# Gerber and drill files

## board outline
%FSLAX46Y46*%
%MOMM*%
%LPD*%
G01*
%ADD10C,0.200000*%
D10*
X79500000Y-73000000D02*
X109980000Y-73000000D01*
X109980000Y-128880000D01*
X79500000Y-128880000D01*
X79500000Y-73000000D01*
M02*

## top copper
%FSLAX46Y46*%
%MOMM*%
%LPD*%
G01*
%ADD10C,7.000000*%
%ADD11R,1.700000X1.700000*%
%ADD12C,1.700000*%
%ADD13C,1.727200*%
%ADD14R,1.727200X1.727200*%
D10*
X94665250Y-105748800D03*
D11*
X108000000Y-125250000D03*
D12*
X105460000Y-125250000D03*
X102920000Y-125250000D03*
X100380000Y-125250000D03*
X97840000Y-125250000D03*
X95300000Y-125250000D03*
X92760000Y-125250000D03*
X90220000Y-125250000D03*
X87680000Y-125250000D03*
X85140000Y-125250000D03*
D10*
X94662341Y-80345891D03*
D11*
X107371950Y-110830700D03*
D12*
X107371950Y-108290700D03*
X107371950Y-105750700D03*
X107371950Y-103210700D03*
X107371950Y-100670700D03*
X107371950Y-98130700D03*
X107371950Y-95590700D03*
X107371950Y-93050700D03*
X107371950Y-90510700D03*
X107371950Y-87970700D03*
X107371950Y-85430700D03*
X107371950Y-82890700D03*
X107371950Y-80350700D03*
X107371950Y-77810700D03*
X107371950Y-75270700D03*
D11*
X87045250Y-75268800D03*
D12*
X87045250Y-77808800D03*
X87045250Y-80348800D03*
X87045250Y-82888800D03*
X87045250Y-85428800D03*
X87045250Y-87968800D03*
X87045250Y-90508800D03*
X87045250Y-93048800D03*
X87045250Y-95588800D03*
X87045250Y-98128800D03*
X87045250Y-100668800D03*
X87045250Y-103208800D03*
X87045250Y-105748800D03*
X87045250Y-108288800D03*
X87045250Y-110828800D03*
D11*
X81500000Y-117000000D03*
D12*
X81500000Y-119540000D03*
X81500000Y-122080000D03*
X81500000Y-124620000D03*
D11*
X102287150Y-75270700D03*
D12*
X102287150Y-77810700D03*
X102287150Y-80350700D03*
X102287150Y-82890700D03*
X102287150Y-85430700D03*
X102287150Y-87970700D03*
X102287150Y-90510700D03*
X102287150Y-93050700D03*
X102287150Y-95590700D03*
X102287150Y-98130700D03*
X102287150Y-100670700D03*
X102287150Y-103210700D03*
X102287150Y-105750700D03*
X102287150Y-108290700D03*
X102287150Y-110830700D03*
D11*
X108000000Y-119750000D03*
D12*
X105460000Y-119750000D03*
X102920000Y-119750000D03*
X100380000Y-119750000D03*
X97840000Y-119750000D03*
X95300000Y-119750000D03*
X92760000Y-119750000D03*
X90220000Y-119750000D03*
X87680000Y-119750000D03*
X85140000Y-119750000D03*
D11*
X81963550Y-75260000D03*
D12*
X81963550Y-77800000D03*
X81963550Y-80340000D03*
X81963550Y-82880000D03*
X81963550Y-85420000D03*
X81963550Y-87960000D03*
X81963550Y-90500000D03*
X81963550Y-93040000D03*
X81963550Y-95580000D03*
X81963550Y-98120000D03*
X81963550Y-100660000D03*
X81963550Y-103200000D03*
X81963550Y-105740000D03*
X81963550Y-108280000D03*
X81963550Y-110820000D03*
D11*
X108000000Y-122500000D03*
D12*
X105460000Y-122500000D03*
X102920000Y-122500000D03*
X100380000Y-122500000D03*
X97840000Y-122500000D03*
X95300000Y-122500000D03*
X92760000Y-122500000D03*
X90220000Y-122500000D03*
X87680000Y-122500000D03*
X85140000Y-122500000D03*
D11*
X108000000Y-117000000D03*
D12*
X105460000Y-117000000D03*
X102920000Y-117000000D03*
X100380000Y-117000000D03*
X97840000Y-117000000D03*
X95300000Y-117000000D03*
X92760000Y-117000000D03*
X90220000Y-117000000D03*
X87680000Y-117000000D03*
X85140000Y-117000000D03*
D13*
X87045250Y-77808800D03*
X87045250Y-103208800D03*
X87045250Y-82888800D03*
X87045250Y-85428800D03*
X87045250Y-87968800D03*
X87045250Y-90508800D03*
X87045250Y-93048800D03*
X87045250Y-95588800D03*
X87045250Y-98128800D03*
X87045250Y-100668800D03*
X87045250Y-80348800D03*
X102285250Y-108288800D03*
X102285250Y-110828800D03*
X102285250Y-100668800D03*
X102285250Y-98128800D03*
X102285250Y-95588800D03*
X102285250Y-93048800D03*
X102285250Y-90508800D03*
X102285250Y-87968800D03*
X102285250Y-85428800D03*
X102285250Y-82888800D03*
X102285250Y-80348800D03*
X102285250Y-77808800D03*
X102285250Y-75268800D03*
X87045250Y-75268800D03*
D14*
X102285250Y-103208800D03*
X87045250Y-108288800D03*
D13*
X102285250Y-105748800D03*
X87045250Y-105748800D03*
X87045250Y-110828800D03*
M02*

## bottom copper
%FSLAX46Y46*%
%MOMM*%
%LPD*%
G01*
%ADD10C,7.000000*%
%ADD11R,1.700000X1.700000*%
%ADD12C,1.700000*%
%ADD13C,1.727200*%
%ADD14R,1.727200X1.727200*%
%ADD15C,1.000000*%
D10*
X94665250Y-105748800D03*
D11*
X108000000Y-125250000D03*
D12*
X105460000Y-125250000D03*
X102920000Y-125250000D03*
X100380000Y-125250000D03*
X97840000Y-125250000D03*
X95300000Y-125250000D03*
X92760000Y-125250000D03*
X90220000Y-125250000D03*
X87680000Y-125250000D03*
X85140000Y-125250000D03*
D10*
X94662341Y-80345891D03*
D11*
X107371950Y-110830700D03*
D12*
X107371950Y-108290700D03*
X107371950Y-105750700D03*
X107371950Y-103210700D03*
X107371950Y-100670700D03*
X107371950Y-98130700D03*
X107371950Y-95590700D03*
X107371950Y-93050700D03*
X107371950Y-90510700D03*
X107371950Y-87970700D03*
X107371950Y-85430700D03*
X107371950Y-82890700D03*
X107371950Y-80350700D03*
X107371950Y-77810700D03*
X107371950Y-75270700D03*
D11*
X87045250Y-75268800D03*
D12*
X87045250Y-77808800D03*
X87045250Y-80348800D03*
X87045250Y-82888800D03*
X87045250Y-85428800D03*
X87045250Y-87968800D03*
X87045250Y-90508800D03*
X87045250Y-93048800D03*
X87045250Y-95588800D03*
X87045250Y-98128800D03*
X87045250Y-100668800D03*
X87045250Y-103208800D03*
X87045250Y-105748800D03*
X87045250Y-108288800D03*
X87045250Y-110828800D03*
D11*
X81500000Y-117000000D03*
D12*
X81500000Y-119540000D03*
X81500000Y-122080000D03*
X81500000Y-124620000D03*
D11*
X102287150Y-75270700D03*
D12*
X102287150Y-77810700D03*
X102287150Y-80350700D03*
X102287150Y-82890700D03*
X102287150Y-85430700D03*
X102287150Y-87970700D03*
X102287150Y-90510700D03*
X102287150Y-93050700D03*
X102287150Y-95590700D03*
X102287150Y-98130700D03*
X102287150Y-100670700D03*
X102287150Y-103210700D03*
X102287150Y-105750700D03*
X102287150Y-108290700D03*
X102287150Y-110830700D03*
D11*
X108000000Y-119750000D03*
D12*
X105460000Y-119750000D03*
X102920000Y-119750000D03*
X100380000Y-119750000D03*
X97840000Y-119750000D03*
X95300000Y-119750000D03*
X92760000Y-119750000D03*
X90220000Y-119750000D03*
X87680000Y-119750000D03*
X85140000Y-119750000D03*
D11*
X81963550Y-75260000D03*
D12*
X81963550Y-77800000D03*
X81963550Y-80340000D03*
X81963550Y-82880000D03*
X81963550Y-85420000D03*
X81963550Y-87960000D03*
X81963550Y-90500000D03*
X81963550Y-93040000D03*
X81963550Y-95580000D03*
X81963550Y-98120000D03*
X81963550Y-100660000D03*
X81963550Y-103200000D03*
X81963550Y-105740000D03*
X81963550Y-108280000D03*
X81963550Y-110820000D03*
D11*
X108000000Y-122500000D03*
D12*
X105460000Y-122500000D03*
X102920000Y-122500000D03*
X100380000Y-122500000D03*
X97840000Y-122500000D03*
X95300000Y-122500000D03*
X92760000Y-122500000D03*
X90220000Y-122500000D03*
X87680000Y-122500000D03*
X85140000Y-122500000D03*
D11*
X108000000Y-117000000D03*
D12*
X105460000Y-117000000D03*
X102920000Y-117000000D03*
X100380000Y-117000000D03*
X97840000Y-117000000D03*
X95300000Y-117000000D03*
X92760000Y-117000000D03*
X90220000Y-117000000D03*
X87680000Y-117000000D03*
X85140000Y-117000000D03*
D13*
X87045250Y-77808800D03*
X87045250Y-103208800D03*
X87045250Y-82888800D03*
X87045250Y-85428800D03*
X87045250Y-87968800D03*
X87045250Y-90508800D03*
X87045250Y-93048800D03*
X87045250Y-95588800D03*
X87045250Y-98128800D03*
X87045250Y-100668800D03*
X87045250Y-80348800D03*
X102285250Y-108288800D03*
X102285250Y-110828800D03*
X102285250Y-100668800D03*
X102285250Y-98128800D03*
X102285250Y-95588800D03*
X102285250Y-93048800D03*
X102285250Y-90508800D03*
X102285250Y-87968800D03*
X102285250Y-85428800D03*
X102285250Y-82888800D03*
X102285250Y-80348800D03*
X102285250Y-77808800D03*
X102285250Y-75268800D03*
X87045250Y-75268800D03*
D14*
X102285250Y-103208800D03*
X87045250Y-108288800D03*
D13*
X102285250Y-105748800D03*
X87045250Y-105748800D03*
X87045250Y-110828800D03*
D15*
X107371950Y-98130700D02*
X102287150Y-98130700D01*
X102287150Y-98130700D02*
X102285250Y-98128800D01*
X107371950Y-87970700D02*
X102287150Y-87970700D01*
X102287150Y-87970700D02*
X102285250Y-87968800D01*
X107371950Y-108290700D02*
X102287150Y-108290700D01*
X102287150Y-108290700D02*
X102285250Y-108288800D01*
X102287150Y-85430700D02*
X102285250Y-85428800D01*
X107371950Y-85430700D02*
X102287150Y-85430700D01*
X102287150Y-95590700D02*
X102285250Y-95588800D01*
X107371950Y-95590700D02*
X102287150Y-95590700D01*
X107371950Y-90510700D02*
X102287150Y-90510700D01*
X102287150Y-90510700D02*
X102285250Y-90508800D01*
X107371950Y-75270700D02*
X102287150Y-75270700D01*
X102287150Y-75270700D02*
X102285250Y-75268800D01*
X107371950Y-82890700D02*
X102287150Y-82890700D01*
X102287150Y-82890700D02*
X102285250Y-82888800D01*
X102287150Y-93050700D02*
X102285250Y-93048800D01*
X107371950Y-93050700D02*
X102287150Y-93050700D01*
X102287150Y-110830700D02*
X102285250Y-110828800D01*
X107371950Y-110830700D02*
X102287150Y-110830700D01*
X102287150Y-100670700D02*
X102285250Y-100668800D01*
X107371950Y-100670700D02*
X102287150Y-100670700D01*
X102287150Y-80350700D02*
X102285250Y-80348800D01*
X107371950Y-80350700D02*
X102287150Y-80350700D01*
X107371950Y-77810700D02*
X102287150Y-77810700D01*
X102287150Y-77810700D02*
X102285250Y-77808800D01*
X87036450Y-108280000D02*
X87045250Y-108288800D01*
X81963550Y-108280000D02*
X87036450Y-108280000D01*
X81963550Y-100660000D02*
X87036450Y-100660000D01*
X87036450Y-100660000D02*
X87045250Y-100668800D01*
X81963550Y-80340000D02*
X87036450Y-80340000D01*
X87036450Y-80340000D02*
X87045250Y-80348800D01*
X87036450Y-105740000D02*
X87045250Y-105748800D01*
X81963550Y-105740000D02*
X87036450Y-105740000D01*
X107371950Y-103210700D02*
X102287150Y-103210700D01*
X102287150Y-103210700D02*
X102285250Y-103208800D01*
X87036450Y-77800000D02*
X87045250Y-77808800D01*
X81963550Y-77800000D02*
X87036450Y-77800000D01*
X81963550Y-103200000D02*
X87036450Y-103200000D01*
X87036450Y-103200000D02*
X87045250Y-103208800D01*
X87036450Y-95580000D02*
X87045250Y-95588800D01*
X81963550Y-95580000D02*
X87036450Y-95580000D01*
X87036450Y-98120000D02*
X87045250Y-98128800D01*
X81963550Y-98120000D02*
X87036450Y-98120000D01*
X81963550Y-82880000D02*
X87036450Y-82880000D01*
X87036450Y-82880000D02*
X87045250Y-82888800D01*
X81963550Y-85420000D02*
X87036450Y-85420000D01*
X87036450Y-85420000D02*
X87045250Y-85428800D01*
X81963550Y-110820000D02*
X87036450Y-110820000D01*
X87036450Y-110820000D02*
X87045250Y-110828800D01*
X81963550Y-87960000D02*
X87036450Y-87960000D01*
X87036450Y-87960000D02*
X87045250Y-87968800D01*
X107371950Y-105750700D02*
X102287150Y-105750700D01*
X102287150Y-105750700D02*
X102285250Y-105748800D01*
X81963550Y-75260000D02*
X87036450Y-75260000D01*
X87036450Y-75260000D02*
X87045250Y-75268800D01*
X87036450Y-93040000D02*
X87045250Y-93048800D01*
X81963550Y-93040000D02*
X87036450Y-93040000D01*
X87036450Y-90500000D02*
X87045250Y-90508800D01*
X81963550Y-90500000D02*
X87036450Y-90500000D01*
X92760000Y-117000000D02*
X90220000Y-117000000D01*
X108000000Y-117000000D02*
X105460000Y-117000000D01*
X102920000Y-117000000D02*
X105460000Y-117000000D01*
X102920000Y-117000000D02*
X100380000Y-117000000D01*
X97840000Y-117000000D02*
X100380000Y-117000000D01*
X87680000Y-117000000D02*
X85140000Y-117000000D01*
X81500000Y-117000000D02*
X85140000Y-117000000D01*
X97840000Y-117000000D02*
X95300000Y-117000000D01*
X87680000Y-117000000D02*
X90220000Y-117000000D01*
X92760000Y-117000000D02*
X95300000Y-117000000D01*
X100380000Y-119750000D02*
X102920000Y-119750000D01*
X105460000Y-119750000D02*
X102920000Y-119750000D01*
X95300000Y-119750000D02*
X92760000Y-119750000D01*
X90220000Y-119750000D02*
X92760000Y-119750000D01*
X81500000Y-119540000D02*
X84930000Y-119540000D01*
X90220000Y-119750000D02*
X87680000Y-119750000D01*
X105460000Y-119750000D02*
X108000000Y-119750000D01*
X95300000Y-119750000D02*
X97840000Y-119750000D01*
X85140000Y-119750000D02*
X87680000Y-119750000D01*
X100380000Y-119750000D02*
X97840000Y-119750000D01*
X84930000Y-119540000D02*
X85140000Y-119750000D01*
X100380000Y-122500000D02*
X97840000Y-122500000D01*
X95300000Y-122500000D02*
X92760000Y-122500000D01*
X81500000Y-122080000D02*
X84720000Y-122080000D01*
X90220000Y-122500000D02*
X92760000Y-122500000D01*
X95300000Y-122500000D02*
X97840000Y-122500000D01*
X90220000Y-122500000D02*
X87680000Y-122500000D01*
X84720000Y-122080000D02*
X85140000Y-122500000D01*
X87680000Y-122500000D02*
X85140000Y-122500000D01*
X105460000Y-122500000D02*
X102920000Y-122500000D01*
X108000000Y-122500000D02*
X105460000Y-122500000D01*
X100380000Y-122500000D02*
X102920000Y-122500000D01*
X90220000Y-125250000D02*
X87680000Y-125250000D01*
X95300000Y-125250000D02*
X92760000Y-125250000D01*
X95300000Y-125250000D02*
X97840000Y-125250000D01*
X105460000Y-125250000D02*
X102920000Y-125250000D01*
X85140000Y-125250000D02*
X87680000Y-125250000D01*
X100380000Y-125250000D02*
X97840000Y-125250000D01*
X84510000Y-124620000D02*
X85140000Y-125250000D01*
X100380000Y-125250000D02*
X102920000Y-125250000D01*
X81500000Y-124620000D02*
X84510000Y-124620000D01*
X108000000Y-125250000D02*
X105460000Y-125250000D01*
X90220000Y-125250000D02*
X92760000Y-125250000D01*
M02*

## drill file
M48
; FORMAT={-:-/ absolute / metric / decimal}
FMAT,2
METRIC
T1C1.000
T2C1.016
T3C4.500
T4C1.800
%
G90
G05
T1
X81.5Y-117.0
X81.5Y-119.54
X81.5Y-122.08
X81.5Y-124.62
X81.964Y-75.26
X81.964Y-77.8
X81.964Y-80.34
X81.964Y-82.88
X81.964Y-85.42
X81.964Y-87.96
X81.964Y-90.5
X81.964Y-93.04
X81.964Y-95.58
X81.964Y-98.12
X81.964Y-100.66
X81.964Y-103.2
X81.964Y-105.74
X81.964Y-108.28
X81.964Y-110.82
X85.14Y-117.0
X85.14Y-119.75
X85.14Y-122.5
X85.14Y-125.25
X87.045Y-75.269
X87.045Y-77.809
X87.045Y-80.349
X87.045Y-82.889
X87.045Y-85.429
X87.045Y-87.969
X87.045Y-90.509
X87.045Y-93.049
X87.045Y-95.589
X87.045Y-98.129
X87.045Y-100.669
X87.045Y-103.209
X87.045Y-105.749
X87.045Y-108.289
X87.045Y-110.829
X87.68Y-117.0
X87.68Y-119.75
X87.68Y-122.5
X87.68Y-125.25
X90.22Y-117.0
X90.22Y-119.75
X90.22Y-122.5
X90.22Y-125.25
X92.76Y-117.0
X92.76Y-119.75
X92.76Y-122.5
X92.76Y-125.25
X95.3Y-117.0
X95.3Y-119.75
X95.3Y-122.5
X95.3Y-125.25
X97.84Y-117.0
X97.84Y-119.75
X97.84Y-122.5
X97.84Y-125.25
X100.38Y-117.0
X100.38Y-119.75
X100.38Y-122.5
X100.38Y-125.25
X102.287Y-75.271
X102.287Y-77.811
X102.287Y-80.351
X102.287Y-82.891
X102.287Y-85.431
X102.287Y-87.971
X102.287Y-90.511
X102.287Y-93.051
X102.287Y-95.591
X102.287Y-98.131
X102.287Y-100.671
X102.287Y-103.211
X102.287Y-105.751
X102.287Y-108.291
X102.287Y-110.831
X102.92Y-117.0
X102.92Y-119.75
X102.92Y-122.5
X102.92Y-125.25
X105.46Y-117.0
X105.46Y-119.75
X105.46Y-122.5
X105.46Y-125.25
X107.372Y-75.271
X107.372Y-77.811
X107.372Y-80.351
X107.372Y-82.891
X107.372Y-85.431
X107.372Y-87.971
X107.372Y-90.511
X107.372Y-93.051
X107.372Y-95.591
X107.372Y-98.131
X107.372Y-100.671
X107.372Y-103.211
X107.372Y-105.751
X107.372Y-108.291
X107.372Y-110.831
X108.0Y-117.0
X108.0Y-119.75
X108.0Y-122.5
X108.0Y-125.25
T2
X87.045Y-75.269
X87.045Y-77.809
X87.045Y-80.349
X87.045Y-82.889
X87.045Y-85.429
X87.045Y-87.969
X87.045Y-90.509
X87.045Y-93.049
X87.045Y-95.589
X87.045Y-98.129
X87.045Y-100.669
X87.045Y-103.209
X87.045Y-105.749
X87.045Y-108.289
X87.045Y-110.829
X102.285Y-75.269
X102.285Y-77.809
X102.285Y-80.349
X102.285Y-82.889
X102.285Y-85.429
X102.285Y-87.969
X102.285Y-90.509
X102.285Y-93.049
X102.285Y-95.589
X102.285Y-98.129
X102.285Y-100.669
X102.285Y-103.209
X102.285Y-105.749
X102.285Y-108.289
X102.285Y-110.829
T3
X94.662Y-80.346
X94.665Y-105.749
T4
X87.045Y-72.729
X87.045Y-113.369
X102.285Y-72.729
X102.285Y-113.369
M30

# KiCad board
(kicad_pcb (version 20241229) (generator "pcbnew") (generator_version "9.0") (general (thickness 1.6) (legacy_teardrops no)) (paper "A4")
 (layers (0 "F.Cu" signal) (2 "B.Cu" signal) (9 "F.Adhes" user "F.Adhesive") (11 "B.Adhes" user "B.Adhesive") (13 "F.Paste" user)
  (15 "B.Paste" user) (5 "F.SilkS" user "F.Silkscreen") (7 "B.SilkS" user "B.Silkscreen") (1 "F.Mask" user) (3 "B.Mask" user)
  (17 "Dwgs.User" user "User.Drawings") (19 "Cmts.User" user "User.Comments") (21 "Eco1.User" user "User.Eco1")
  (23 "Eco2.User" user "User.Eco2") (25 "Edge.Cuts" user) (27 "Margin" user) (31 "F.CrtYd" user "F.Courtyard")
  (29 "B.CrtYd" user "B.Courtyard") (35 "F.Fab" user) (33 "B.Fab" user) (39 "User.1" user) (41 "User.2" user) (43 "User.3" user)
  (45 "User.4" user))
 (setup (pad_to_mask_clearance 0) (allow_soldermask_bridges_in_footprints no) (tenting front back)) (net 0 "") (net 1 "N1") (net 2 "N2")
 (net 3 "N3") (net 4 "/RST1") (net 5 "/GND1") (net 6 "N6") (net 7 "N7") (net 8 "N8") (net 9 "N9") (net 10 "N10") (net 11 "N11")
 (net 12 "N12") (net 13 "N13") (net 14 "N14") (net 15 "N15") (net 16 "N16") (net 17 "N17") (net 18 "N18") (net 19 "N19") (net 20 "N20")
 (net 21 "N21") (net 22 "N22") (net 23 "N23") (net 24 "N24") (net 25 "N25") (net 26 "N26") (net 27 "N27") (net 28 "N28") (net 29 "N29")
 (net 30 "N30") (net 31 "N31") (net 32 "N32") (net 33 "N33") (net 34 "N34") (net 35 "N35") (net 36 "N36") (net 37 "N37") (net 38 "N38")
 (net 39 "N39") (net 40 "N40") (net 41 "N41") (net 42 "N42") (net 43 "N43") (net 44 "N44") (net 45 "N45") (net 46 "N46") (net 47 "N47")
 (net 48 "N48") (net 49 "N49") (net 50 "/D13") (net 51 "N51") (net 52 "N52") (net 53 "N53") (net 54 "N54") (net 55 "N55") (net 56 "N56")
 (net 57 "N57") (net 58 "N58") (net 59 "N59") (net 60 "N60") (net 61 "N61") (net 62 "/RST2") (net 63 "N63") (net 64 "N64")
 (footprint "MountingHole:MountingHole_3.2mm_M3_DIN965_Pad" (layer "F.Cu") (at 94.66525 105.7488)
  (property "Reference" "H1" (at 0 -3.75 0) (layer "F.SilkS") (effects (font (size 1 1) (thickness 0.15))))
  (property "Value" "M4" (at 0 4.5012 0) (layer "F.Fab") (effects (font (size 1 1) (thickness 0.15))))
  (pad "1" thru_hole circle (at 0 0) (size 7 7) (drill 4.5) (layers "*.Cu" "*.Mask") (remove_unused_layers no) (zone_connect 2)))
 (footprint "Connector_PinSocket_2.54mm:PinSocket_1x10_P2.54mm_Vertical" (layer "F.Cu") (at 108 125.25 -90)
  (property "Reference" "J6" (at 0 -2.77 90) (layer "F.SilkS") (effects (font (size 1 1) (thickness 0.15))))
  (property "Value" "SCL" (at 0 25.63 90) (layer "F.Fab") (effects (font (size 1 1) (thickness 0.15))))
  (pad "1" thru_hole rect (at 0 0 270) (size 1.7 1.7) (drill 1) (layers "*.Cu" "*.Mask") (remove_unused_layers no) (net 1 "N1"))
  (pad "2" thru_hole circle (at 0 2.54 270) (size 1.7 1.7) (drill 1) (layers "*.Cu" "*.Mask") (remove_unused_layers no) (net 1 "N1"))
  (pad "3" thru_hole circle (at 0 5.08 270) (size 1.7 1.7) (drill 1) (layers "*.Cu" "*.Mask") (remove_unused_layers no) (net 1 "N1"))
  (pad "4" thru_hole circle (at 0 7.62 270) (size 1.7 1.7) (drill 1) (layers "*.Cu" "*.Mask") (remove_unused_layers no) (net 1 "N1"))
  (pad "5" thru_hole circle (at 0 10.16 270) (size 1.7 1.7) (drill 1) (layers "*.Cu" "*.Mask") (remove_unused_layers no) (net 1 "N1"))
  (pad "6" thru_hole circle (at 0 12.7 270) (size 1.7 1.7) (drill 1) (layers "*.Cu" "*.Mask") (remove_unused_layers no) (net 1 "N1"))
  (pad "7" thru_hole circle (at 0 15.24 270) (size 1.7 1.7) (drill 1) (layers "*.Cu" "*.Mask") (remove_unused_layers no) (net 1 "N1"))
  (pad "8" thru_hole circle (at 0 17.78 270) (size 1.7 1.7) (drill 1) (layers "*.Cu" "*.Mask") (remove_unused_layers no) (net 1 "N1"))
  (pad "9" thru_hole circle (at 0 20.32 270) (size 1.7 1.7) (drill 1) (layers "*.Cu" "*.Mask") (remove_unused_layers no) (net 1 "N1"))
  (pad "10" thru_hole circle (at 0 22.86 270) (size 1.7 1.7) (drill 1) (layers "*.Cu" "*.Mask") (remove_unused_layers no) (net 1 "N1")))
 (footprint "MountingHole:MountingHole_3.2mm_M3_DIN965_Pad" (layer "F.Cu") (at 94.662341 80.345891)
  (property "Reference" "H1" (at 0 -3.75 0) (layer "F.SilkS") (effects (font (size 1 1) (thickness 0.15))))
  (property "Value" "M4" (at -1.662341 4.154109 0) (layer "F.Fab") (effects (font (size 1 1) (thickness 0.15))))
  (pad "1" thru_hole circle (at 0 0) (size 7 7) (drill 4.5) (layers "*.Cu" "*.Mask") (remove_unused_layers no) (zone_connect 2)))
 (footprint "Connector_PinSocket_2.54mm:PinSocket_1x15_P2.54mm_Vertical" (layer "F.Cu") (at 107.37195 110.8307 180)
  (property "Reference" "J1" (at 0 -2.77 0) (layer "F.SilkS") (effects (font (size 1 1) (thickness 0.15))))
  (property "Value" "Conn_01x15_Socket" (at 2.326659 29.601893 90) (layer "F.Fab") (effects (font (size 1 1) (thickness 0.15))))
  (pad "1" thru_hole rect (at 0 0 180) (size 1.7 1.7) (drill 1) (layers "*.Cu" "*.Mask") (remove_unused_layers no) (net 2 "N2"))
  (pad "2" thru_hole circle (at 0 2.54 180) (size 1.7 1.7) (drill 1) (layers "*.Cu" "*.Mask") (remove_unused_layers no) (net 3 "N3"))
  (pad "3" thru_hole circle (at 0 5.08 180) (size 1.7 1.7) (drill 1) (layers "*.Cu" "*.Mask") (remove_unused_layers no) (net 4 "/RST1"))
  (pad "4" thru_hole circle (at 0 7.62 180) (size 1.7 1.7) (drill 1) (layers "*.Cu" "*.Mask") (remove_unused_layers no) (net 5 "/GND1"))
  (pad "5" thru_hole circle (at 0 10.16 180) (size 1.7 1.7) (drill 1) (layers "*.Cu" "*.Mask") (remove_unused_layers no) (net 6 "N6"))
  (pad "6" thru_hole circle (at 0 12.7 180) (size 1.7 1.7) (drill 1) (layers "*.Cu" "*.Mask") (remove_unused_layers no) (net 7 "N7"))
  (pad "7" thru_hole circle (at 0 15.24 180) (size 1.7 1.7) (drill 1) (layers "*.Cu" "*.Mask") (remove_unused_layers no) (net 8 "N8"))
  (pad "8" thru_hole circle (at 0 17.78 180) (size 1.7 1.7) (drill 1) (layers "*.Cu" "*.Mask") (remove_unused_layers no) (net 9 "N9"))
  (pad "9" thru_hole circle (at 0 20.32 180) (size 1.7 1.7) (drill 1) (layers "*.Cu" "*.Mask") (remove_unused_layers no) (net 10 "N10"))
  (pad "10" thru_hole circle (at 0 22.86 180) (size 1.7 1.7) (drill 1) (layers "*.Cu" "*.Mask") (remove_unused_layers no) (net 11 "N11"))
  (pad "11" thru_hole circle (at 0 25.4 180) (size 1.7 1.7) (drill 1) (layers "*.Cu" "*.Mask") (remove_unused_layers no) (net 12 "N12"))
  (pad "12" thru_hole circle (at 0 27.94 180) (size 1.7 1.7) (drill 1) (layers "*.Cu" "*.Mask") (remove_unused_layers no) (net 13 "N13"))
  (pad "13" thru_hole circle (at 0 30.48 180) (size 1.7 1.7) (drill 1) (layers "*.Cu" "*.Mask") (remove_unused_layers no) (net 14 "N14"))
  (pad "14" thru_hole circle (at 0 33.02 180) (size 1.7 1.7) (drill 1) (layers "*.Cu" "*.Mask") (remove_unused_layers no) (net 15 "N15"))
  (pad "15" thru_hole circle (at 0 35.56 180) (size 1.7 1.7) (drill 1) (layers "*.Cu" "*.Mask") (remove_unused_layers no) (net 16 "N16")))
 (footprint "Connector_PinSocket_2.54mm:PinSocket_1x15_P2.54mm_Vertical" (layer "F.Cu") (at 87.04525 75.2688)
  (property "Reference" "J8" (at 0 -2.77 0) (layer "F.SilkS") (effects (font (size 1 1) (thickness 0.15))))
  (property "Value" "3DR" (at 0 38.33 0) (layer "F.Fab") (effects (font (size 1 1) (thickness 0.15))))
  (pad "1" thru_hole rect (at 0 0) (size 1.7 1.7) (drill 1) (layers "*.Cu" "*.Mask") (remove_unused_layers no) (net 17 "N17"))
  (pad "2" thru_hole circle (at 0 2.54) (size 1.7 1.7) (drill 1) (layers "*.Cu" "*.Mask") (remove_unused_layers no) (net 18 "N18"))
  (pad "3" thru_hole circle (at 0 5.08) (size 1.7 1.7) (drill 1) (layers "*.Cu" "*.Mask") (remove_unused_layers no) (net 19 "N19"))
  (pad "4" thru_hole circle (at 0 7.62) (size 1.7 1.7) (drill 1) (layers "*.Cu" "*.Mask") (remove_unused_layers no) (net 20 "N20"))
  (pad "5" thru_hole circle (at 0 10.16) (size 1.7 1.7) (drill 1) (layers "*.Cu" "*.Mask") (remove_unused_layers no) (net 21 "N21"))
  (pad "6" thru_hole circle (at 0 12.7) (size 1.7 1.7) (drill 1) (layers "*.Cu" "*.Mask") (remove_unused_layers no) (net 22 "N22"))
  (pad "7" thru_hole circle (at 0 15.24) (size 1.7 1.7) (drill 1) (layers "*.Cu" "*.Mask") (remove_unused_layers no) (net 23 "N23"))
  (pad "8" thru_hole circle (at 0 17.78) (size 1.7 1.7) (drill 1) (layers "*.Cu" "*.Mask") (remove_unused_layers no) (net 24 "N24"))
  (pad "9" thru_hole circle (at 0 20.32) (size 1.7 1.7) (drill 1) (layers "*.Cu" "*.Mask") (remove_unused_layers no) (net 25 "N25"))
  (pad "10" thru_hole circle (at 0 22.86) (size 1.7 1.7) (drill 1) (layers "*.Cu" "*.Mask") (remove_unused_layers no) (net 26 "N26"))
  (pad "11" thru_hole circle (at 0 25.4) (size 1.7 1.7) (drill 1) (layers "*.Cu" "*.Mask") (remove_unused_layers no) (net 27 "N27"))
  (pad "12" thru_hole circle (at 0 27.94) (size 1.7 1.7) (drill 1) (layers "*.Cu" "*.Mask") (remove_unused_layers no) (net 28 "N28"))
  (pad "13" thru_hole circle (at 0 30.48) (size 1.7 1.7) (drill 1) (layers "*.Cu" "*.Mask") (remove_unused_layers no) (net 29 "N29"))
  (pad "14" thru_hole circle (at 0 33.02) (size 1.7 1.7) (drill 1) (layers "*.Cu" "*.Mask") (remove_unused_layers no) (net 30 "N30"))
  (pad "15" thru_hole circle (at 0 35.56) (size 1.7 1.7) (drill 1) (layers "*.Cu" "*.Mask") (remove_unused_layers no) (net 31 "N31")))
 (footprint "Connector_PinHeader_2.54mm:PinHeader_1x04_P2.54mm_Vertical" (layer "F.Cu") (at 81.5 117)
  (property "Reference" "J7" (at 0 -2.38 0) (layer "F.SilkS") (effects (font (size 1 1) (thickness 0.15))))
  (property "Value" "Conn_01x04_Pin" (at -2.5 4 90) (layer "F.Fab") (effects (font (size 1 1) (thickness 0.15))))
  (pad "1" thru_hole rect (at 0 0) (size 1.7 1.7) (drill 1) (layers "*.Cu" "*.Mask") (remove_unused_layers no) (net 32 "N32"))
  (pad "2" thru_hole circle (at 0 2.54) (size 1.7 1.7) (drill 1) (layers "*.Cu" "*.Mask") (remove_unused_layers no) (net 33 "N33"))
  (pad "3" thru_hole circle (at 0 5.08) (size 1.7 1.7) (drill 1) (layers "*.Cu" "*.Mask") (remove_unused_layers no) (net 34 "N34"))
  (pad "4" thru_hole circle (at 0 7.62) (size 1.7 1.7) (drill 1) (layers "*.Cu" "*.Mask") (remove_unused_layers no) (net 1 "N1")))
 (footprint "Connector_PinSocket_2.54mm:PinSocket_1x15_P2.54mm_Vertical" (layer "F.Cu") (at 102.28715 75.2707)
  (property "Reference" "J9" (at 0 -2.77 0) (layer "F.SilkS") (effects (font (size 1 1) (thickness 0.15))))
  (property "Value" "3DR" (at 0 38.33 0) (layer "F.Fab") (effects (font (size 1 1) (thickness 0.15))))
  (pad "1" thru_hole rect (at 0 0) (size 1.7 1.7) (drill 1) (layers "*.Cu" "*.Mask") (remove_unused_layers no) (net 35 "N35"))
  (pad "2" thru_hole circle (at 0 2.54) (size 1.7 1.7) (drill 1) (layers "*.Cu" "*.Mask") (remove_unused_layers no) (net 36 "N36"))
  (pad "3" thru_hole circle (at 0 5.08) (size 1.7 1.7) (drill 1) (layers "*.Cu" "*.Mask") (remove_unused_layers no) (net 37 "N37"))
  (pad "4" thru_hole circle (at 0 7.62) (size 1.7 1.7) (drill 1) (layers "*.Cu" "*.Mask") (remove_unused_layers no) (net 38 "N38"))
  (pad "5" thru_hole circle (at 0 10.16) (size 1.7 1.7) (drill 1) (layers "*.Cu" "*.Mask") (remove_unused_layers no) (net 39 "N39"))
  (pad "6" thru_hole circle (at 0 12.7) (size 1.7 1.7) (drill 1) (layers "*.Cu" "*.Mask") (remove_unused_layers no) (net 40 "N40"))
  (pad "7" thru_hole circle (at 0 15.24) (size 1.7 1.7) (drill 1) (layers "*.Cu" "*.Mask") (remove_unused_layers no) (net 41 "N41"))
  (pad "8" thru_hole circle (at 0 17.78) (size 1.7 1.7) (drill 1) (layers "*.Cu" "*.Mask") (remove_unused_layers no) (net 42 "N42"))
  (pad "9" thru_hole circle (at 0 20.32) (size 1.7 1.7) (drill 1) (layers "*.Cu" "*.Mask") (remove_unused_layers no) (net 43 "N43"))
  (pad "10" thru_hole circle (at 0 22.86) (size 1.7 1.7) (drill 1) (layers "*.Cu" "*.Mask") (remove_unused_layers no) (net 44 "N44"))
  (pad "11" thru_hole circle (at 0 25.4) (size 1.7 1.7) (drill 1) (layers "*.Cu" "*.Mask") (remove_unused_layers no) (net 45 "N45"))
  (pad "12" thru_hole circle (at 0 27.94) (size 1.7 1.7) (drill 1) (layers "*.Cu" "*.Mask") (remove_unused_layers no) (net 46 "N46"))
  (pad "13" thru_hole circle (at 0 30.48) (size 1.7 1.7) (drill 1) (layers "*.Cu" "*.Mask") (remove_unused_layers no) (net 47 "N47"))
  (pad "14" thru_hole circle (at 0 33.02) (size 1.7 1.7) (drill 1) (layers "*.Cu" "*.Mask") (remove_unused_layers no) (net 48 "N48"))
  (pad "15" thru_hole circle (at 0 35.56) (size 1.7 1.7) (drill 1) (layers "*.Cu" "*.Mask") (remove_unused_layers no) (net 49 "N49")))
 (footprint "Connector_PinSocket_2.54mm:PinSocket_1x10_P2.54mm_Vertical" (layer "F.Cu") (at 108 119.75 -90)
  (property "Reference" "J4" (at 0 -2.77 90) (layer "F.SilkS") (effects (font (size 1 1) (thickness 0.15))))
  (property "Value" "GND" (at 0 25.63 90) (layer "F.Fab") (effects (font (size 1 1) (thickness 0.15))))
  (pad "1" thru_hole rect (at 0 0 270) (size 1.7 1.7) (drill 1) (layers "*.Cu" "*.Mask") (remove_unused_layers no) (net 33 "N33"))
  (pad "2" thru_hole circle (at 0 2.54 270) (size 1.7 1.7) (drill 1) (layers "*.Cu" "*.Mask") (remove_unused_layers no) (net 33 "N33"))
  (pad "3" thru_hole circle (at 0 5.08 270) (size 1.7 1.7) (drill 1) (layers "*.Cu" "*.Mask") (remove_unused_layers no) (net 33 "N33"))
  (pad "4" thru_hole circle (at 0 7.62 270) (size 1.7 1.7) (drill 1) (layers "*.Cu" "*.Mask") (remove_unused_layers no) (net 33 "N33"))
  (pad "5" thru_hole circle (at 0 10.16 270) (size 1.7 1.7) (drill 1) (layers "*.Cu" "*.Mask") (remove_unused_layers no) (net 33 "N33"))
  (pad "6" thru_hole circle (at 0 12.7 270) (size 1.7 1.7) (drill 1) (layers "*.Cu" "*.Mask") (remove_unused_layers no) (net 33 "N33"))
  (pad "7" thru_hole circle (at 0 15.24 270) (size 1.7 1.7) (drill 1) (layers "*.Cu" "*.Mask") (remove_unused_layers no) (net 33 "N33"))
  (pad "8" thru_hole circle (at 0 17.78 270) (size 1.7 1.7) (drill 1) (layers "*.Cu" "*.Mask") (remove_unused_layers no) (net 33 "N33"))
  (pad "9" thru_hole circle (at 0 20.32 270) (size 1.7 1.7) (drill 1) (layers "*.Cu" "*.Mask") (remove_unused_layers no) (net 33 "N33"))
  (pad "10" thru_hole circle (at 0 22.86 270) (size 1.7 1.7) (drill 1) (layers "*.Cu" "*.Mask") (remove_unused_layers no) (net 33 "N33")))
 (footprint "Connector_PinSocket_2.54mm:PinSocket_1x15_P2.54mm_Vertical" (layer "F.Cu") (at 81.96355 75.26)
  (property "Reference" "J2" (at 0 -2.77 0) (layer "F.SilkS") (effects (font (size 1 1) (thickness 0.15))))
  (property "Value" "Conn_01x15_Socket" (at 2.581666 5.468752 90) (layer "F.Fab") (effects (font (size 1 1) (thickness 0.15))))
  (pad "1" thru_hole rect (at 0 0) (size 1.7 1.7) (drill 1) (layers "*.Cu" "*.Mask") (remove_unused_layers no) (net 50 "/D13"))
  (pad "2" thru_hole circle (at 0 2.54) (size 1.7 1.7) (drill 1) (layers "*.Cu" "*.Mask") (remove_unused_layers no) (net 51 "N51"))
  (pad "3" thru_hole circle (at 0 5.08) (size 1.7 1.7) (drill 1) (layers "*.Cu" "*.Mask") (remove_unused_layers no) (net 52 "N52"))
  (pad "4" thru_hole circle (at 0 7.62) (size 1.7 1.7) (drill 1) (layers "*.Cu" "*.Mask") (remove_unused_layers no) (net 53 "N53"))
  (pad "5" thru_hole circle (at 0 10.16) (size 1.7 1.7) (drill 1) (layers "*.Cu" "*.Mask") (remove_unused_layers no) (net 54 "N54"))
  (pad "6" thru_hole circle (at 0 12.7) (size 1.7 1.7) (drill 1) (layers "*.Cu" "*.Mask") (remove_unused_layers no) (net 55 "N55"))
  (pad "7" thru_hole circle (at 0 15.24) (size 1.7 1.7) (drill 1) (layers "*.Cu" "*.Mask") (remove_unused_layers no) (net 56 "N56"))
  (pad "8" thru_hole circle (at 0 17.78) (size 1.7 1.7) (drill 1) (layers "*.Cu" "*.Mask") (remove_unused_layers no) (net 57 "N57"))
  (pad "9" thru_hole circle (at 0 20.32) (size 1.7 1.7) (drill 1) (layers "*.Cu" "*.Mask") (remove_unused_layers no) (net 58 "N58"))
  (pad "10" thru_hole circle (at 0 22.86) (size 1.7 1.7) (drill 1) (layers "*.Cu" "*.Mask") (remove_unused_layers no) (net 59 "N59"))
  (pad "11" thru_hole circle (at 0 25.4) (size 1.7 1.7) (drill 1) (layers "*.Cu" "*.Mask") (remove_unused_layers no) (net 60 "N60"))
  (pad "12" thru_hole circle (at 0 27.94) (size 1.7 1.7) (drill 1) (layers "*.Cu" "*.Mask") (remove_unused_layers no) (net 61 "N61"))
  (pad "13" thru_hole circle (at 0 30.48) (size 1.7 1.7) (drill 1) (layers "*.Cu" "*.Mask") (remove_unused_layers no) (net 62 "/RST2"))
  (pad "14" thru_hole circle (at 0 33.02) (size 1.7 1.7) (drill 1) (layers "*.Cu" "*.Mask") (remove_unused_layers no) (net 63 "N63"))
  (pad "15" thru_hole circle (at 0 35.56) (size 1.7 1.7) (drill 1) (layers "*.Cu" "*.Mask") (remove_unused_layers no) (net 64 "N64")))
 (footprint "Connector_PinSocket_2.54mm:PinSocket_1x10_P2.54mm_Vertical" (layer "F.Cu") (at 108 122.5 -90)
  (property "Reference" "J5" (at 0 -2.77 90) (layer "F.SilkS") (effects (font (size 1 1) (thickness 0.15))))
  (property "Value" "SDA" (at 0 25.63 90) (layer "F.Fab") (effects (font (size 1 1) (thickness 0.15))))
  (pad "1" thru_hole rect (at 0 0 270) (size 1.7 1.7) (drill 1) (layers "*.Cu" "*.Mask") (remove_unused_layers no) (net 34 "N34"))
  (pad "2" thru_hole circle (at 0 2.54 270) (size 1.7 1.7) (drill 1) (layers "*.Cu" "*.Mask") (remove_unused_layers no) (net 34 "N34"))
  (pad "3" thru_hole circle (at 0 5.08 270) (size 1.7 1.7) (drill 1) (layers "*.Cu" "*.Mask") (remove_unused_layers no) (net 34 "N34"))
  (pad "4" thru_hole circle (at 0 7.62 270) (size 1.7 1.7) (drill 1) (layers "*.Cu" "*.Mask") (remove_unused_layers no) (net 34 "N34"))
  (pad "5" thru_hole circle (at 0 10.16 270) (size 1.7 1.7) (drill 1) (layers "*.Cu" "*.Mask") (remove_unused_layers no) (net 34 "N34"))
  (pad "6" thru_hole circle (at 0 12.7 270) (size 1.7 1.7) (drill 1) (layers "*.Cu" "*.Mask") (remove_unused_layers no) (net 34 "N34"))
  (pad "7" thru_hole circle (at 0 15.24 270) (size 1.7 1.7) (drill 1) (layers "*.Cu" "*.Mask") (remove_unused_layers no) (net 34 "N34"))
  (pad "8" thru_hole circle (at 0 17.78 270) (size 1.7 1.7) (drill 1) (layers "*.Cu" "*.Mask") (remove_unused_layers no) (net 34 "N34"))
  (pad "9" thru_hole circle (at 0 20.32 270) (size 1.7 1.7) (drill 1) (layers "*.Cu" "*.Mask") (remove_unused_layers no) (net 34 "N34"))
  (pad "10" thru_hole circle (at 0 22.86 270) (size 1.7 1.7) (drill 1) (layers "*.Cu" "*.Mask") (remove_unused_layers no) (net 34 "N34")))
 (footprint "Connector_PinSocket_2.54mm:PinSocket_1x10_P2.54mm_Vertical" (layer "F.Cu") (at 108 117 -90)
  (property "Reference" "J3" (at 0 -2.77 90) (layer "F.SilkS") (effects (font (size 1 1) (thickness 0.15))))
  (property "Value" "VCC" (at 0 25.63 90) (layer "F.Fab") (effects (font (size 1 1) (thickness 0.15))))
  (pad "1" thru_hole rect (at 0 0 270) (size 1.7 1.7) (drill 1) (layers "*.Cu" "*.Mask") (remove_unused_layers no) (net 32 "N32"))
  (pad "2" thru_hole circle (at 0 2.54 270) (size 1.7 1.7) (drill 1) (layers "*.Cu" "*.Mask") (remove_unused_layers no) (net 32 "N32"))
  (pad "3" thru_hole circle (at 0 5.08 270) (size 1.7 1.7) (drill 1) (layers "*.Cu" "*.Mask") (remove_unused_layers no) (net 32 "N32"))
  (pad "4" thru_hole circle (at 0 7.62 270) (size 1.7 1.7) (drill 1) (layers "*.Cu" "*.Mask") (remove_unused_layers no) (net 32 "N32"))
  (pad "5" thru_hole circle (at 0 10.16 270) (size 1.7 1.7) (drill 1) (layers "*.Cu" "*.Mask") (remove_unused_layers no) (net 32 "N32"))
  (pad "6" thru_hole circle (at 0 12.7 270) (size 1.7 1.7) (drill 1) (layers "*.Cu" "*.Mask") (remove_unused_layers no) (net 32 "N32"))
  (pad "7" thru_hole circle (at 0 15.24 270) (size 1.7 1.7) (drill 1) (layers "*.Cu" "*.Mask") (remove_unused_layers no) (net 32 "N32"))
  (pad "8" thru_hole circle (at 0 17.78 270) (size 1.7 1.7) (drill 1) (layers "*.Cu" "*.Mask") (remove_unused_layers no) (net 32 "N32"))
  (pad "9" thru_hole circle (at 0 20.32 270) (size 1.7 1.7) (drill 1) (layers "*.Cu" "*.Mask") (remove_unused_layers no) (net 32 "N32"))
  (pad "10" thru_hole circle (at 0 22.86 270) (size 1.7 1.7) (drill 1) (layers "*.Cu" "*.Mask") (remove_unused_layers no) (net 32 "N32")))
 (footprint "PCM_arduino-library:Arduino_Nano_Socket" (layer "F.Cu") (at 94.66525 71.4588 180)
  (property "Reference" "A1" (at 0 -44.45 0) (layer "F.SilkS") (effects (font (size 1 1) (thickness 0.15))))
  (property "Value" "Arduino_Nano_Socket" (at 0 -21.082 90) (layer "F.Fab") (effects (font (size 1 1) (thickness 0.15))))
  (pad "" np_thru_hole circle (at -7.62 -41.91 180) (size 1.8 1.8) (drill 1.8) (layers "*.Cu" "*.Mask"))
  (pad "" np_thru_hole circle (at -7.62 -1.27 180) (size 1.8 1.8) (drill 1.8) (layers "*.Cu" "*.Mask"))
  (pad "" np_thru_hole circle (at 7.62 -41.91 180) (size 1.8 1.8) (drill 1.8) (layers "*.Cu" "*.Mask"))
  (pad "" np_thru_hole circle (at 7.62 -1.27 180) (size 1.8 1.8) (drill 1.8) (layers "*.Cu" "*.Mask"))
  (pad "3V3" thru_hole circle (at 7.62 -6.35 180) (size 1.7272 1.7272) (drill 1.016) (layers "*.Cu" "*.Mask") (remove_unused_layers no)
   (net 51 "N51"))
  (pad "5V" thru_hole circle (at 7.62 -31.75 180) (size 1.7272 1.7272) (drill 1.016) (layers "*.Cu" "*.Mask") (remove_unused_layers no)
   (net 61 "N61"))
  (pad "A0" thru_hole circle (at 7.62 -11.43 180) (size 1.7272 1.7272) (drill 1.016) (layers "*.Cu" "*.Mask") (remove_unused_layers no)
   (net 53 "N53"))
  (pad "A1" thru_hole circle (at 7.62 -13.97 180) (size 1.7272 1.7272) (drill 1.016) (layers "*.Cu" "*.Mask") (remove_unused_layers no)
   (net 54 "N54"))
  (pad "A2" thru_hole circle (at 7.62 -16.51 180) (size 1.7272 1.7272) (drill 1.016) (layers "*.Cu" "*.Mask") (remove_unused_layers no)
   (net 55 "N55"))
  (pad "A3" thru_hole circle (at 7.62 -19.05 180) (size 1.7272 1.7272) (drill 1.016) (layers "*.Cu" "*.Mask") (remove_unused_layers no)
   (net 56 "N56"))
  (pad "A4" thru_hole circle (at 7.62 -21.59 180) (size 1.7272 1.7272) (drill 1.016) (layers "*.Cu" "*.Mask") (remove_unused_layers no)
   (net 57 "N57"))
  (pad "A5" thru_hole circle (at 7.62 -24.13 180) (size 1.7272 1.7272) (drill 1.016) (layers "*.Cu" "*.Mask") (remove_unused_layers no)
   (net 58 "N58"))
  (pad "A6" thru_hole circle (at 7.62 -26.67 180) (size 1.7272 1.7272) (drill 1.016) (layers "*.Cu" "*.Mask") (remove_unused_layers no)
   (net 59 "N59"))
  (pad "A7" thru_hole circle (at 7.62 -29.21 180) (size 1.7272 1.7272) (drill 1.016) (layers "*.Cu" "*.Mask") (remove_unused_layers no)
   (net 60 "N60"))
  (pad "AREF" thru_hole circle (at 7.62 -8.89 180) (size 1.7272 1.7272) (drill 1.016) (layers "*.Cu" "*.Mask") (remove_unused_layers no)
   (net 52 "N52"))
  (pad "D0" thru_hole circle (at -7.62 -36.83 180) (size 1.7272 1.7272) (drill 1.016) (layers "*.Cu" "*.Mask") (remove_unused_layers no)
   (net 3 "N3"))
  (pad "D1" thru_hole circle (at -7.62 -39.37 180) (size 1.7272 1.7272) (drill 1.016) (layers "*.Cu" "*.Mask") (remove_unused_layers no)
   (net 2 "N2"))
  (pad "D2" thru_hole circle (at -7.62 -29.21 180) (size 1.7272 1.7272) (drill 1.016) (layers "*.Cu" "*.Mask") (remove_unused_layers no)
   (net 6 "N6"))
  (pad "D3" thru_hole circle (at -7.62 -26.67 180) (size 1.7272 1.7272) (drill 1.016) (layers "*.Cu" "*.Mask") (remove_unused_layers no)
   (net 7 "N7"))
  (pad "D4" thru_hole circle (at -7.62 -24.13 180) (size 1.7272 1.7272) (drill 1.016) (layers "*.Cu" "*.Mask") (remove_unused_layers no)
   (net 8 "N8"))
  (pad "D5" thru_hole circle (at -7.62 -21.59 180) (size 1.7272 1.7272) (drill 1.016) (layers "*.Cu" "*.Mask") (remove_unused_layers no)
   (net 9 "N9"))
  (pad "D6" thru_hole circle (at -7.62 -19.05 180) (size 1.7272 1.7272) (drill 1.016) (layers "*.Cu" "*.Mask") (remove_unused_layers no)
   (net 10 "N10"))
  (pad "D7" thru_hole circle (at -7.62 -16.51 180) (size 1.7272 1.7272) (drill 1.016) (layers "*.Cu" "*.Mask") (remove_unused_layers no)
   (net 11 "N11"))
  (pad "D8" thru_hole circle (at -7.62 -13.97 180) (size 1.7272 1.7272) (drill 1.016) (layers "*.Cu" "*.Mask") (remove_unused_layers no)
   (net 12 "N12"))
  (pad "D9" thru_hole circle (at -7.62 -11.43 180) (size 1.7272 1.7272) (drill 1.016) (layers "*.Cu" "*.Mask") (remove_unused_layers no)
   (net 13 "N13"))
  (pad "D10" thru_hole circle (at -7.62 -8.89 180) (size 1.7272 1.7272) (drill 1.016) (layers "*.Cu" "*.Mask") (remove_unused_layers no)
   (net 14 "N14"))
  (pad "D11" thru_hole circle (at -7.62 -6.35 180) (size 1.7272 1.7272) (drill 1.016) (layers "*.Cu" "*.Mask") (remove_unused_layers no)
   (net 15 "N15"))
  (pad "D12" thru_hole circle (at -7.62 -3.81 180) (size 1.7272 1.7272) (drill 1.016) (layers "*.Cu" "*.Mask") (remove_unused_layers no)
   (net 16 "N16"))
  (pad "D13" thru_hole circle (at 7.62 -3.81 180) (size 1.7272 1.7272) (drill 1.016) (layers "*.Cu" "*.Mask") (remove_unused_layers no)
   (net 50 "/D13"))
  (pad "GND1" thru_hole rect (at -7.62 -31.75 180) (size 1.7272 1.7272) (drill 1.016) (layers "*.Cu" "*.Mask") (remove_unused_layers no)
   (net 5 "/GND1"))
  (pad "GND2" thru_hole rect (at 7.62 -36.83 180) (size 1.7272 1.7272) (drill 1.016) (layers "*.Cu" "*.Mask") (remove_unused_layers no)
   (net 63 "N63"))
  (pad "RST1" thru_hole circle (at -7.62 -34.29 180) (size 1.7272 1.7272) (drill 1.016) (layers "*.Cu" "*.Mask") (remove_unused_layers no)
   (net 4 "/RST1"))
  (pad "RST2" thru_hole circle (at 7.62 -34.29 180) (size 1.7272 1.7272) (drill 1.016) (layers "*.Cu" "*.Mask") (remove_unused_layers no)
   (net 62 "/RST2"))
  (pad "VIN" thru_hole circle (at 7.62 -39.37 180) (size 1.7272 1.7272) (drill 1.016) (layers "*.Cu" "*.Mask") (remove_unused_layers no)
   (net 64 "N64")))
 (gr_rect (start 79.5 73) (end 109.98 128.88) (stroke (width 0.2) (type solid)) (fill no) (layer "Edge.Cuts"))
 (segment (start 107.37195 98.1307) (end 102.28715 98.1307) (width 1) (layer "B.Cu") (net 7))
 (segment (start 102.28715 98.1307) (end 102.28525 98.1288) (width 1) (layer "B.Cu") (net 7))
 (segment (start 107.37195 87.9707) (end 102.28715 87.9707) (width 1) (layer "B.Cu") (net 11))
 (segment (start 102.28715 87.9707) (end 102.28525 87.9688) (width 1) (layer "B.Cu") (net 11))
 (segment (start 107.37195 108.2907) (end 102.28715 108.2907) (width 1) (layer "B.Cu") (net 3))
 (segment (start 102.28715 108.2907) (end 102.28525 108.2888) (width 1) (layer "B.Cu") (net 3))
 (segment (start 102.28715 85.4307) (end 102.28525 85.4288) (width 1) (layer "B.Cu") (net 12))
 (segment (start 107.37195 85.4307) (end 102.28715 85.4307) (width 1) (layer "B.Cu") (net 12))
 (segment (start 102.28715 95.5907) (end 102.28525 95.5888) (width 1) (layer "B.Cu") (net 8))
 (segment (start 107.37195 95.5907) (end 102.28715 95.5907) (width 1) (layer "B.Cu") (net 8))
 (segment (start 107.37195 90.5107) (end 102.28715 90.5107) (width 1) (layer "B.Cu") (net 10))
 (segment (start 102.28715 90.5107) (end 102.28525 90.5088) (width 1) (layer "B.Cu") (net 10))
 (segment (start 107.37195 75.2707) (end 102.28715 75.2707) (width 1) (layer "B.Cu") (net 16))
 (segment (start 102.28715 75.2707) (end 102.28525 75.2688) (width 1) (layer "B.Cu") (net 16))
 (segment (start 107.37195 82.8907) (end 102.28715 82.8907) (width 1) (layer "B.Cu") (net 13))
 (segment (start 102.28715 82.8907) (end 102.28525 82.8888) (width 1) (layer "B.Cu") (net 13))
 (segment (start 102.28715 93.0507) (end 102.28525 93.0488) (width 1) (layer "B.Cu") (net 9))
 (segment (start 107.37195 93.0507) (end 102.28715 93.0507) (width 1) (layer "B.Cu") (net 9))
 (segment (start 102.28715 110.8307) (end 102.28525 110.8288) (width 1) (layer "B.Cu") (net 2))
 (segment (start 107.37195 110.8307) (end 102.28715 110.8307) (width 1) (layer "B.Cu") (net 2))
 (segment (start 102.28715 100.6707) (end 102.28525 100.6688) (width 1) (layer "B.Cu") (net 6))
 (segment (start 107.37195 100.6707) (end 102.28715 100.6707) (width 1) (layer "B.Cu") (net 6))
 (segment (start 102.28715 80.3507) (end 102.28525 80.3488) (width 1) (layer "B.Cu") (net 14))
 (segment (start 107.37195 80.3507) (end 102.28715 80.3507) (width 1) (layer "B.Cu") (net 14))
 (segment (start 107.37195 77.8107) (end 102.28715 77.8107) (width 1) (layer "B.Cu") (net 15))
 (segment (start 102.28715 77.8107) (end 102.28525 77.8088) (width 1) (layer "B.Cu") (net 15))
 (segment (start 87.03645 108.28) (end 87.04525 108.2888) (width 1) (layer "B.Cu") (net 63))
 (segment (start 81.96355 108.28) (end 87.03645 108.28) (width 1) (layer "B.Cu") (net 63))
 (segment (start 81.96355 100.66) (end 87.03645 100.66) (width 1) (layer "B.Cu") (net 60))
 (segment (start 87.03645 100.66) (end 87.04525 100.6688) (width 1) (layer "B.Cu") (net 60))
 (segment (start 81.96355 80.34) (end 87.03645 80.34) (width 1) (layer "B.Cu") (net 52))
 (segment (start 87.03645 80.34) (end 87.04525 80.3488) (width 1) (layer "B.Cu") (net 52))
 (segment (start 87.03645 105.74) (end 87.04525 105.7488) (width 1) (layer "B.Cu") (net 62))
 (segment (start 81.96355 105.74) (end 87.03645 105.74) (width 1) (layer "B.Cu") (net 62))
 (segment (start 107.37195 103.2107) (end 102.28715 103.2107) (width 1) (layer "B.Cu") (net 5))
 (segment (start 102.28715 103.2107) (end 102.28525 103.2088) (width 1) (layer "B.Cu") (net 5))
 (segment (start 87.03645 77.8) (end 87.04525 77.8088) (width 1) (layer "B.Cu") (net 51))
 (segment (start 81.96355 77.8) (end 87.03645 77.8) (width 1) (layer "B.Cu") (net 51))
 (segment (start 81.96355 103.2) (end 87.03645 103.2) (width 1) (layer "B.Cu") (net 61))
 (segment (start 87.03645 103.2) (end 87.04525 103.2088) (width 1) (layer "B.Cu") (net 61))
 (segment (start 87.03645 95.58) (end 87.04525 95.5888) (width 1) (layer "B.Cu") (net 58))
 (segment (start 81.96355 95.58) (end 87.03645 95.58) (width 1) (layer "B.Cu") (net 58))
 (segment (start 87.03645 98.12) (end 87.04525 98.1288) (width 1) (layer "B.Cu") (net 59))
 (segment (start 81.96355 98.12) (end 87.03645 98.12) (width 1) (layer "B.Cu") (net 59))
 (segment (start 81.96355 82.88) (end 87.03645 82.88) (width 1) (layer "B.Cu") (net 53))
 (segment (start 87.03645 82.88) (end 87.04525 82.8888) (width 1) (layer "B.Cu") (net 53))
 (segment (start 81.96355 85.42) (end 87.03645 85.42) (width 1) (layer "B.Cu") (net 54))
 (segment (start 87.03645 85.42) (end 87.04525 85.4288) (width 1) (layer "B.Cu") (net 54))
 (segment (start 81.96355 110.82) (end 87.03645 110.82) (width 1) (layer "B.Cu") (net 64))
 (segment (start 87.03645 110.82) (end 87.04525 110.8288) (width 1) (layer "B.Cu") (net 64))
 (segment (start 81.96355 87.96) (end 87.03645 87.96) (width 1) (layer "B.Cu") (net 55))
 (segment (start 87.03645 87.96) (end 87.04525 87.9688) (width 1) (layer "B.Cu") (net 55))
 (segment (start 107.37195 105.7507) (end 102.28715 105.7507) (width 1) (layer "B.Cu") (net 4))
 (segment (start 102.28715 105.7507) (end 102.28525 105.7488) (width 1) (layer "B.Cu") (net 4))
 (segment (start 81.96355 75.26) (end 87.03645 75.26) (width 1) (layer "B.Cu") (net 50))
 (segment (start 87.03645 75.26) (end 87.04525 75.2688) (width 1) (layer "B.Cu") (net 50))
 (segment (start 87.03645 93.04) (end 87.04525 93.0488) (width 1) (layer "B.Cu") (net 57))
 (segment (start 81.96355 93.04) (end 87.03645 93.04) (width 1) (layer "B.Cu") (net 57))
 (segment (start 87.03645 90.5) (end 87.04525 90.5088) (width 1) (layer "B.Cu") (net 56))
 (segment (start 81.96355 90.5) (end 87.03645 90.5) (width 1) (layer "B.Cu") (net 56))
 (segment (start 92.76 117) (end 90.22 117) (width 1) (layer "B.Cu") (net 32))
 (segment (start 108 117) (end 105.46 117) (width 1) (layer "B.Cu") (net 32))
 (segment (start 102.92 117) (end 105.46 117) (width 1) (layer "B.Cu") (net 32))
 (segment (start 102.92 117) (end 100.38 117) (width 1) (layer "B.Cu") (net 32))
 (segment (start 97.84 117) (end 100.38 117) (width 1) (layer "B.Cu") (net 32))
 (segment (start 87.68 117) (end 85.14 117) (width 1) (layer "B.Cu") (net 32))
 (segment (start 81.5 117) (end 85.14 117) (width 1) (layer "B.Cu") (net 32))
 (segment (start 97.84 117) (end 95.3 117) (width 1) (layer "B.Cu") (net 32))
 (segment (start 87.68 117) (end 90.22 117) (width 1) (layer "B.Cu") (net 32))
 (segment (start 92.76 117) (end 95.3 117) (width 1) (layer "B.Cu") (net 32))
 (segment (start 100.38 119.75) (end 102.92 119.75) (width 1) (layer "B.Cu") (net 33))
 (segment (start 105.46 119.75) (end 102.92 119.75) (width 1) (layer "B.Cu") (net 33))
 (segment (start 95.3 119.75) (end 92.76 119.75) (width 1) (layer "B.Cu") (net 33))
 (segment (start 90.22 119.75) (end 92.76 119.75) (width 1) (layer "B.Cu") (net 33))
 (segment (start 81.5 119.54) (end 84.93 119.54) (width 1) (layer "B.Cu") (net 33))
 (segment (start 90.22 119.75) (end 87.68 119.75) (width 1) (layer "B.Cu") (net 33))
 (segment (start 105.46 119.75) (end 108 119.75) (width 1) (layer "B.Cu") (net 33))
 (segment (start 95.3 119.75) (end 97.84 119.75) (width 1) (layer "B.Cu") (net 33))
 (segment (start 85.14 119.75) (end 87.68 119.75) (width 1) (layer "B.Cu") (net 33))
 (segment (start 100.38 119.75) (end 97.84 119.75) (width 1) (layer "B.Cu") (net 33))
 (segment (start 84.93 119.54) (end 85.14 119.75) (width 1) (layer "B.Cu") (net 33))
 (segment (start 100.38 122.5) (end 97.84 122.5) (width 1) (layer "B.Cu") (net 34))
 (segment (start 95.3 122.5) (end 92.76 122.5) (width 1) (layer "B.Cu") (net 34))
 (segment (start 81.5 122.08) (end 84.72 122.08) (width 1) (layer "B.Cu") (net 34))
 (segment (start 90.22 122.5) (end 92.76 122.5) (width 1) (layer "B.Cu") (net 34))
 (segment (start 95.3 122.5) (end 97.84 122.5) (width 1) (layer "B.Cu") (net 34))
 (segment (start 90.22 122.5) (end 87.68 122.5) (width 1) (layer "B.Cu") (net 34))
 (segment (start 84.72 122.08) (end 85.14 122.5) (width 1) (layer "B.Cu") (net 34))
 (segment (start 87.68 122.5) (end 85.14 122.5) (width 1) (layer "B.Cu") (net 34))
 (segment (start 105.46 122.5) (end 102.92 122.5) (width 1) (layer "B.Cu") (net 34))
 (segment (start 108 122.5) (end 105.46 122.5) (width 1) (layer "B.Cu") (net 34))
 (segment (start 100.38 122.5) (end 102.92 122.5) (width 1) (layer "B.Cu") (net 34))
 (segment (start 90.22 125.25) (end 87.68 125.25) (width 1) (layer "B.Cu") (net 1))
 (segment (start 95.3 125.25) (end 92.76 125.25) (width 1) (layer "B.Cu") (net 1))
 (segment (start 95.3 125.25) (end 97.84 125.25) (width 1) (layer "B.Cu") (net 1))
 (segment (start 105.46 125.25) (end 102.92 125.25) (width 1) (layer "B.Cu") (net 1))
 (segment (start 85.14 125.25) (end 87.68 125.25) (width 1) (layer "B.Cu") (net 1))
 (segment (start 100.38 125.25) (end 97.84 125.25) (width 1) (layer "B.Cu") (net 1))
 (segment (start 84.51 124.62) (end 85.14 125.25) (width 1) (layer "B.Cu") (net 1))
 (segment (start 100.38 125.25) (end 102.92 125.25) (width 1) (layer "B.Cu") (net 1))
 (segment (start 81.5 124.62) (end 84.51 124.62) (width 1) (layer "B.Cu") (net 1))
 (segment (start 108 125.25) (end 105.46 125.25) (width 1) (layer "B.Cu") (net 1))
 (segment (start 90.22 125.25) (end 92.76 125.25) (width 1) (layer "B.Cu") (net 1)))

